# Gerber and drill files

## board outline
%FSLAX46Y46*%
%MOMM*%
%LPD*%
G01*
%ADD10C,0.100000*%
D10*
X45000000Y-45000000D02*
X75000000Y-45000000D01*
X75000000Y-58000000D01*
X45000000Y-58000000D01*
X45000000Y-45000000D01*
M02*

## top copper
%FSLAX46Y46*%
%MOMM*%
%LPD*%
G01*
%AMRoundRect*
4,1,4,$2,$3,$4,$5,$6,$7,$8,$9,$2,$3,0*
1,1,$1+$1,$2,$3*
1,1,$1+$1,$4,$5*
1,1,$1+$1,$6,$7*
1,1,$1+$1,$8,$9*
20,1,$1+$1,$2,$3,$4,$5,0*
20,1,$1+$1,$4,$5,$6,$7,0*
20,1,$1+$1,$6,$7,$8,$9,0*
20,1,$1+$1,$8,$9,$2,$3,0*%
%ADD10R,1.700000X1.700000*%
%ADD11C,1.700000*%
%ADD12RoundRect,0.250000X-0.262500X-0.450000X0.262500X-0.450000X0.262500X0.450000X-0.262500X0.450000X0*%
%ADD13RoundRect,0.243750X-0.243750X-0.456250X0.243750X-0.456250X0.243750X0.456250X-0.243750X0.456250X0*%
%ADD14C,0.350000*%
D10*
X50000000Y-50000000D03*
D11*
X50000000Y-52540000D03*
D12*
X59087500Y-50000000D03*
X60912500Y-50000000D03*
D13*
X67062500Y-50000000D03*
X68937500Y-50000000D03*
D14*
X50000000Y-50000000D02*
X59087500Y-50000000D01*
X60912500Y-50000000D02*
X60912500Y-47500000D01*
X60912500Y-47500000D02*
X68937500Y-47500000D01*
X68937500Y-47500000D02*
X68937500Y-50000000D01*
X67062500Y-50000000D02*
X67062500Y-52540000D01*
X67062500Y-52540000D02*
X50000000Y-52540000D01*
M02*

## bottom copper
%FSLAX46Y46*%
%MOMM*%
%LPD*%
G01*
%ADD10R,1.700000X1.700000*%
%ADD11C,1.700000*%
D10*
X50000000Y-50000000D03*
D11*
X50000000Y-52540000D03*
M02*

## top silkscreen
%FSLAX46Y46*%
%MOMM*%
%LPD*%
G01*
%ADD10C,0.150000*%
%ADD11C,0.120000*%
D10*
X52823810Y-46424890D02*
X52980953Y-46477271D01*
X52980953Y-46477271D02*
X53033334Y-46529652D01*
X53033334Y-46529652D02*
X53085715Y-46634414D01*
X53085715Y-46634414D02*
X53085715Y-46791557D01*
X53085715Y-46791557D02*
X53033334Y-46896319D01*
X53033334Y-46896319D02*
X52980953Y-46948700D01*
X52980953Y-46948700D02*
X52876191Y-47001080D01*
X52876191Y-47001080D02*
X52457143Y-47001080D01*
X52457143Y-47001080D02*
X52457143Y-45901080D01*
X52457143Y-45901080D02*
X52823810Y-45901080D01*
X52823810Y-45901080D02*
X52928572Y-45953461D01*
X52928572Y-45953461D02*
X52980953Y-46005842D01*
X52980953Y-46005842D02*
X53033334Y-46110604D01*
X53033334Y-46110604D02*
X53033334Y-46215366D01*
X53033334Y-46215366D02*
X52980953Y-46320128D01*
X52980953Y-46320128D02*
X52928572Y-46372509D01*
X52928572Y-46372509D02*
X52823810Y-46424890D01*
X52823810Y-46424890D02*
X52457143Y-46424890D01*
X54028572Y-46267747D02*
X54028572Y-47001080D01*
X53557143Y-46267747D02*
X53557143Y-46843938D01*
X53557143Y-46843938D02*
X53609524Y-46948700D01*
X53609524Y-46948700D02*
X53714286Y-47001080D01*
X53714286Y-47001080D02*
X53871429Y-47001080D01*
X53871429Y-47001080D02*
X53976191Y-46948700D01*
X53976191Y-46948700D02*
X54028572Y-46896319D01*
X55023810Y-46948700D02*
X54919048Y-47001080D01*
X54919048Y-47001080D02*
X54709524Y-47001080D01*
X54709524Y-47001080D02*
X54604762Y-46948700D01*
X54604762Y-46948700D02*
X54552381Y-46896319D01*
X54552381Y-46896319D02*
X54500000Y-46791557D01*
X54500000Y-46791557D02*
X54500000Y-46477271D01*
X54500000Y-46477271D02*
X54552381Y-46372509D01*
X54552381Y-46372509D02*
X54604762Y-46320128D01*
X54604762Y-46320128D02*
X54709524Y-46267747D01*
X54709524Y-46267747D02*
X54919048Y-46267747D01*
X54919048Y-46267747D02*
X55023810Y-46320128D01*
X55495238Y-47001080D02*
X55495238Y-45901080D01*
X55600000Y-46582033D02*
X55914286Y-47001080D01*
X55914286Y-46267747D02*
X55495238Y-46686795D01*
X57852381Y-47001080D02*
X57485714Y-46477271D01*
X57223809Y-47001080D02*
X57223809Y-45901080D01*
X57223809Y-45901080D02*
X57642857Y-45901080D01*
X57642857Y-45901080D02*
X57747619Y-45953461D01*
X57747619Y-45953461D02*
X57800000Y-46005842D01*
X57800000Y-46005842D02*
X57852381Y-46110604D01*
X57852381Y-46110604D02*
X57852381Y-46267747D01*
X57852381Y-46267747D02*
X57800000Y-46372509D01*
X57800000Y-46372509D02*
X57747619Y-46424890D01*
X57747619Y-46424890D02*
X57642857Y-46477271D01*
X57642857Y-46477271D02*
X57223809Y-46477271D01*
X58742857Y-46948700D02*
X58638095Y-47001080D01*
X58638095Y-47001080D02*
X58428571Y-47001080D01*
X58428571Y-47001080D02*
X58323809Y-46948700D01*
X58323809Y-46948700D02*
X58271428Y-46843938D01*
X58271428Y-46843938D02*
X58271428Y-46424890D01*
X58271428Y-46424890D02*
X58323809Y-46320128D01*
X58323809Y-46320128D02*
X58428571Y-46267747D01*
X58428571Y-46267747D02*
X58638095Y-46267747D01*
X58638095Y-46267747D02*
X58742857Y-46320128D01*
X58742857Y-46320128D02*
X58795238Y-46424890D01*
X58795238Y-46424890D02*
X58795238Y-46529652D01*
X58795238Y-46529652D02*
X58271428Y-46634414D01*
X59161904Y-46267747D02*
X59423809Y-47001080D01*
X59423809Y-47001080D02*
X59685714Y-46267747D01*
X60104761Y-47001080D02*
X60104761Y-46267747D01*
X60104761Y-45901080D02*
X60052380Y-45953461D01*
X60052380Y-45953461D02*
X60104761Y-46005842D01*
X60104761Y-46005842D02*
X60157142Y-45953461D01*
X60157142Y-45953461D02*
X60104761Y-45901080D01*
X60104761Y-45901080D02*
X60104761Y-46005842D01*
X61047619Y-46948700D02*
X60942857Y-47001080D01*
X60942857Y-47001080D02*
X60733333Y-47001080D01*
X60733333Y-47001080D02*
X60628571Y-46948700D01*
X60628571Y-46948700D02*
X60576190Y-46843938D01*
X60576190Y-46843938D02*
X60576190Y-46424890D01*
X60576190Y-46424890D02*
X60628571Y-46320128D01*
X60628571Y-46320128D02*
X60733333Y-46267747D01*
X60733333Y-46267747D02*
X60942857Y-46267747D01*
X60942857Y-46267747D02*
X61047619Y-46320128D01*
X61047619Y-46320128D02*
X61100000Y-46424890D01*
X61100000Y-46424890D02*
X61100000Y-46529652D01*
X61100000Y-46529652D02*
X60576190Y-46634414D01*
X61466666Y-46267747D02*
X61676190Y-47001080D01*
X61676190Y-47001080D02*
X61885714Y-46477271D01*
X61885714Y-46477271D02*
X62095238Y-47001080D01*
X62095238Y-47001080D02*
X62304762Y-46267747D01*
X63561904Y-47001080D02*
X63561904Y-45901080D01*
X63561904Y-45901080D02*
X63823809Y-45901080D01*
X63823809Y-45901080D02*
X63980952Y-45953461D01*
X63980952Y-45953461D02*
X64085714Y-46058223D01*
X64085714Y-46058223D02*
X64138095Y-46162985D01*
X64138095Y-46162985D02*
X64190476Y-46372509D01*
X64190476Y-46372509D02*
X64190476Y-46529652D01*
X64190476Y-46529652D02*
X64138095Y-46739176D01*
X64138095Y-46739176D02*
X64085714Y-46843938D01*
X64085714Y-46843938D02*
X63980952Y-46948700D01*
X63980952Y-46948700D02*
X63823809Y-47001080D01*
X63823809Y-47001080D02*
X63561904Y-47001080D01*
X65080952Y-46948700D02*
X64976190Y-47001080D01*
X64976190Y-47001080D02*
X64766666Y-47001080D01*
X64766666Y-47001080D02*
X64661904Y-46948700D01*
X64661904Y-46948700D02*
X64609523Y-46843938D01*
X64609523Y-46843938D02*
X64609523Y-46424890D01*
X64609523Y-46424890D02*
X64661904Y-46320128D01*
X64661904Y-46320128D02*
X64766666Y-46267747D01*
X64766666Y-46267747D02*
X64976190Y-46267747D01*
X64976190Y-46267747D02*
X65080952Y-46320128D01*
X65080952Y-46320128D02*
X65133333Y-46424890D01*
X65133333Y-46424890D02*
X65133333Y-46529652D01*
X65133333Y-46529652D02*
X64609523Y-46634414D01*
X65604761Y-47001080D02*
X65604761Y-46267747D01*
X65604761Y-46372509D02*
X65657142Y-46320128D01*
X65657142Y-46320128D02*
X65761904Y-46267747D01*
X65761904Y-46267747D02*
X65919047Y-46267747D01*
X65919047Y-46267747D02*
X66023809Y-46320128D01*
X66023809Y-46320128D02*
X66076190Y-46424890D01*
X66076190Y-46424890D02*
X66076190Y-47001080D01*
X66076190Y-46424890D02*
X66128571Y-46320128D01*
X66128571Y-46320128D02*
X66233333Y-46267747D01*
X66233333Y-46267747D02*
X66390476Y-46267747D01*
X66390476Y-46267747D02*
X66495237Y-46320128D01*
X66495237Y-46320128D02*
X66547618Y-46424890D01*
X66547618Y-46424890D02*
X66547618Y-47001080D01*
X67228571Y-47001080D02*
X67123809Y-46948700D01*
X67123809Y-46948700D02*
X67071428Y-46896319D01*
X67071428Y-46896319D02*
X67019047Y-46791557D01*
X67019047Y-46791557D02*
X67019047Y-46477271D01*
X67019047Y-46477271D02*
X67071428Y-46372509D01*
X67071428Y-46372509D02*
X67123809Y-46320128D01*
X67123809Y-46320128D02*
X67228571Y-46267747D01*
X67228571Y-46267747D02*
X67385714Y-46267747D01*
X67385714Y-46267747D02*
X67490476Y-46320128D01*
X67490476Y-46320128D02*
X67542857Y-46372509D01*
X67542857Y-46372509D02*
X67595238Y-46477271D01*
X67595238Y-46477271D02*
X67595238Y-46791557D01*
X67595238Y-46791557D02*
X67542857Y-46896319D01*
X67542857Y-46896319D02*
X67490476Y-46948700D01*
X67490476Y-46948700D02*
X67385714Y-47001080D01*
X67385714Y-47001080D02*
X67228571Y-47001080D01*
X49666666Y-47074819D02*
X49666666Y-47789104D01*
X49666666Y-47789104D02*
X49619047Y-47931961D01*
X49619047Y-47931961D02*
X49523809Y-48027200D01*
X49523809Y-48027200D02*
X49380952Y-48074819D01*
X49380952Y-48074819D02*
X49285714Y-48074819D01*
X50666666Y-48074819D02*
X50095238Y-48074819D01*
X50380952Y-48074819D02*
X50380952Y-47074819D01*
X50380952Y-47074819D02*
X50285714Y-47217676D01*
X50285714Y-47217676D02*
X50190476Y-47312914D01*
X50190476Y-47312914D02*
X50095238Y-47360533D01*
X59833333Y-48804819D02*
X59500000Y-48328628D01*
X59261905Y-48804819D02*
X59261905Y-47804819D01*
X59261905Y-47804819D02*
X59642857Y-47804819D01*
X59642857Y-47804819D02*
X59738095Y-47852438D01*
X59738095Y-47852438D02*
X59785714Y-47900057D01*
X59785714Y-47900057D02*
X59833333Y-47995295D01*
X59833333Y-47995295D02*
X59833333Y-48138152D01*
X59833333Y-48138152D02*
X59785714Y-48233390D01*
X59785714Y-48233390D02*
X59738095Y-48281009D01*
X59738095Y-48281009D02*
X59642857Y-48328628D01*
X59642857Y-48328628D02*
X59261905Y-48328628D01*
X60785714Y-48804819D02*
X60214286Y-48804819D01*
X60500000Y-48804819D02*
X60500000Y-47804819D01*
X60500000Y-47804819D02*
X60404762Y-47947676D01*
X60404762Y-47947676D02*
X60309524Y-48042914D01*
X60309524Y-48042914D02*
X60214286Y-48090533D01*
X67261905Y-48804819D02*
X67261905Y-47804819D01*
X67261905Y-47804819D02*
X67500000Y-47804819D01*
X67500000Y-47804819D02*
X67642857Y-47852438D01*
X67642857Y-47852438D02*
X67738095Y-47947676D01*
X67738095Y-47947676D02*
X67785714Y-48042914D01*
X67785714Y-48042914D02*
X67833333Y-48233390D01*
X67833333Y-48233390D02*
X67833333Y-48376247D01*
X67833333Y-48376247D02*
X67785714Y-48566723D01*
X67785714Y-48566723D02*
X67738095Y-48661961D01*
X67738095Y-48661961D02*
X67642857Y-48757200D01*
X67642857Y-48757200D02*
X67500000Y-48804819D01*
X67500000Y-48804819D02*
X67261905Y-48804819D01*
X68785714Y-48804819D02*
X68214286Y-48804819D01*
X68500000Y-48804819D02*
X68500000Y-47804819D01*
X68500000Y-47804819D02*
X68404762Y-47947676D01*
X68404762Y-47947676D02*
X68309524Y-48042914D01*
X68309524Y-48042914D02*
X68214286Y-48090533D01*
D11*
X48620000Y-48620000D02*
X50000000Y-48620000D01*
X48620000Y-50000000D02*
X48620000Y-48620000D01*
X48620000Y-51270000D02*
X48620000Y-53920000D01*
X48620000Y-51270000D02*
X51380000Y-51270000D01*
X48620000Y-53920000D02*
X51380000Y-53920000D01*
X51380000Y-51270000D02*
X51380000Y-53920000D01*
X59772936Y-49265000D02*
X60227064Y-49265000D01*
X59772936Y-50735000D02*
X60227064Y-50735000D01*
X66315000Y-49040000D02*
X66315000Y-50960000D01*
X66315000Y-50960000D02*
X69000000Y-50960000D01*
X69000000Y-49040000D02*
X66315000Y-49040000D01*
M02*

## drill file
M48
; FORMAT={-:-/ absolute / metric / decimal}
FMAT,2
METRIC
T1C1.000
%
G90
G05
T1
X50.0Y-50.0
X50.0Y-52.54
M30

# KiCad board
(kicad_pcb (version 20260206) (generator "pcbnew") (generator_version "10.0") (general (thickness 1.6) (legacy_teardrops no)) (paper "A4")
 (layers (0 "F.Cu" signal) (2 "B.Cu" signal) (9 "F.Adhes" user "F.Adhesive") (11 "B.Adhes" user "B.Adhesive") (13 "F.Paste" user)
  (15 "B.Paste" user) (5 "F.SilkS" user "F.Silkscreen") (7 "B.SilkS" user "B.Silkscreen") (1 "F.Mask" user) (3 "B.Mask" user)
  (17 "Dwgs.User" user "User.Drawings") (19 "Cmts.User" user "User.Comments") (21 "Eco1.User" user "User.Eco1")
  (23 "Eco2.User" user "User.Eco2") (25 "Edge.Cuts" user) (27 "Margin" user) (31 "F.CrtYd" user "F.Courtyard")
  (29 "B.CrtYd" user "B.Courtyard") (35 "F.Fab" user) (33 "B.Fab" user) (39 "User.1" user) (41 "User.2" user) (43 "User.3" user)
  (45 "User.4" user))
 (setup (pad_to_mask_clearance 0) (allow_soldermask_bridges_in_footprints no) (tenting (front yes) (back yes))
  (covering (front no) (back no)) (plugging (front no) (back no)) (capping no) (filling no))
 (gr_rect (start 45 45) (end 75 58) (stroke (width 0.1) (type solid)) (fill no) (layer "Edge.Cuts"))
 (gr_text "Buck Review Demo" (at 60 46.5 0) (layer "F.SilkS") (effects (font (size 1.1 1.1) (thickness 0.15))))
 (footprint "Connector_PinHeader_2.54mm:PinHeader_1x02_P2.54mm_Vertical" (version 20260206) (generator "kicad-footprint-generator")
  (layer "F.Cu") (at 50 50 0)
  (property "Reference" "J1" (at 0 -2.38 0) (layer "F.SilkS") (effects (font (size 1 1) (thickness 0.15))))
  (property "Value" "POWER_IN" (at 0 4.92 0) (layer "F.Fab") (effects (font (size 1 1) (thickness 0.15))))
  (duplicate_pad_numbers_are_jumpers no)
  (fp_line (start -1.38 -1.38) (end 0 -1.38) (stroke (width 0.12) (type solid)) (layer "F.SilkS"))
  (fp_line (start -1.38 0) (end -1.38 -1.38) (stroke (width 0.12) (type solid)) (layer "F.SilkS"))
  (fp_line (start -1.38 1.27) (end -1.38 3.92) (stroke (width 0.12) (type solid)) (layer "F.SilkS"))
  (fp_line (start -1.38 1.27) (end 1.38 1.27) (stroke (width 0.12) (type solid)) (layer "F.SilkS"))
  (fp_line (start -1.38 3.92) (end 1.38 3.92) (stroke (width 0.12) (type solid)) (layer "F.SilkS"))
  (fp_line (start 1.38 1.27) (end 1.38 3.92) (stroke (width 0.12) (type solid)) (layer "F.SilkS"))
  (pad "1" thru_hole rect (at 0 0) (size 1.7 1.7) (drill 1) (layers "*.Cu" "*.Mask") (remove_unused_layers no) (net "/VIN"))
  (pad "2" thru_hole circle (at 0 2.54) (size 1.7 1.7) (drill 1) (layers "*.Cu" "*.Mask") (remove_unused_layers no) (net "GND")))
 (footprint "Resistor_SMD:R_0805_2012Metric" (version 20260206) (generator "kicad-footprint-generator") (layer "F.Cu") (at 60 50 0)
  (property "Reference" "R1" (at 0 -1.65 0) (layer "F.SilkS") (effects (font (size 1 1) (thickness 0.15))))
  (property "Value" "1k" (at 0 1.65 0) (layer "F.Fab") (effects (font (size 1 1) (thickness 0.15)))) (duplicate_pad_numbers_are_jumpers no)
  (fp_line (start -0.227064 -0.735) (end 0.227064 -0.735) (stroke (width 0.12) (type solid)) (layer "F.SilkS"))
  (fp_line (start -0.227064 0.735) (end 0.227064 0.735) (stroke (width 0.12) (type solid)) (layer "F.SilkS"))
  (pad "1" smd roundrect (at -0.9125 0) (size 1.025 1.4) (layers "F.Cu" "F.Mask" "F.Paste") (roundrect_rratio 0.243902) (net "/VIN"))
  (pad "2" smd roundrect (at 0.9125 0) (size 1.025 1.4) (layers "F.Cu" "F.Mask" "F.Paste") (roundrect_rratio 0.243902) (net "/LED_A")))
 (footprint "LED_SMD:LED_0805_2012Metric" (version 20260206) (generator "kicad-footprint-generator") (layer "F.Cu") (at 68 50 0)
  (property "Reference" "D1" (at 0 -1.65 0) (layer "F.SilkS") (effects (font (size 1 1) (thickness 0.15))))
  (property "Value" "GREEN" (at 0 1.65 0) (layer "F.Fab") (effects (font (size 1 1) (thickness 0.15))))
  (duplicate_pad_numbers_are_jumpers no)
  (fp_line (start -1.685 -0.96) (end -1.685 0.96) (stroke (width 0.12) (type solid)) (layer "F.SilkS"))
  (fp_line (start -1.685 0.96) (end 1 0.96) (stroke (width 0.12) (type solid)) (layer "F.SilkS"))
  (fp_line (start 1 -0.96) (end -1.685 -0.96) (stroke (width 0.12) (type solid)) (layer "F.SilkS"))
  (pad "1" smd roundrect (at -0.9375 0) (size 0.975 1.4) (layers "F.Cu" "F.Mask" "F.Paste") (roundrect_rratio 0.25) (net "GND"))
  (pad "2" smd roundrect (at 0.9375 0) (size 0.975 1.4) (layers "F.Cu" "F.Mask" "F.Paste") (roundrect_rratio 0.25) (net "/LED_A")))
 (segment (start 50 50) (end 59.0875 50) (width 0.35) (layer "F.Cu") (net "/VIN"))
 (segment (start 60.9125 50) (end 60.9125 47.5) (width 0.35) (layer "F.Cu") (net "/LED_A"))
 (segment (start 60.9125 47.5) (end 68.9375 47.5) (width 0.35) (layer "F.Cu") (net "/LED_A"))
 (segment (start 68.9375 47.5) (end 68.9375 50) (width 0.35) (layer "F.Cu") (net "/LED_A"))
 (segment (start 67.0625 50) (end 67.0625 52.54) (width 0.35) (layer "F.Cu") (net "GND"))
 (segment (start 67.0625 52.54) (end 50 52.54) (width 0.35) (layer "F.Cu") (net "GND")))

